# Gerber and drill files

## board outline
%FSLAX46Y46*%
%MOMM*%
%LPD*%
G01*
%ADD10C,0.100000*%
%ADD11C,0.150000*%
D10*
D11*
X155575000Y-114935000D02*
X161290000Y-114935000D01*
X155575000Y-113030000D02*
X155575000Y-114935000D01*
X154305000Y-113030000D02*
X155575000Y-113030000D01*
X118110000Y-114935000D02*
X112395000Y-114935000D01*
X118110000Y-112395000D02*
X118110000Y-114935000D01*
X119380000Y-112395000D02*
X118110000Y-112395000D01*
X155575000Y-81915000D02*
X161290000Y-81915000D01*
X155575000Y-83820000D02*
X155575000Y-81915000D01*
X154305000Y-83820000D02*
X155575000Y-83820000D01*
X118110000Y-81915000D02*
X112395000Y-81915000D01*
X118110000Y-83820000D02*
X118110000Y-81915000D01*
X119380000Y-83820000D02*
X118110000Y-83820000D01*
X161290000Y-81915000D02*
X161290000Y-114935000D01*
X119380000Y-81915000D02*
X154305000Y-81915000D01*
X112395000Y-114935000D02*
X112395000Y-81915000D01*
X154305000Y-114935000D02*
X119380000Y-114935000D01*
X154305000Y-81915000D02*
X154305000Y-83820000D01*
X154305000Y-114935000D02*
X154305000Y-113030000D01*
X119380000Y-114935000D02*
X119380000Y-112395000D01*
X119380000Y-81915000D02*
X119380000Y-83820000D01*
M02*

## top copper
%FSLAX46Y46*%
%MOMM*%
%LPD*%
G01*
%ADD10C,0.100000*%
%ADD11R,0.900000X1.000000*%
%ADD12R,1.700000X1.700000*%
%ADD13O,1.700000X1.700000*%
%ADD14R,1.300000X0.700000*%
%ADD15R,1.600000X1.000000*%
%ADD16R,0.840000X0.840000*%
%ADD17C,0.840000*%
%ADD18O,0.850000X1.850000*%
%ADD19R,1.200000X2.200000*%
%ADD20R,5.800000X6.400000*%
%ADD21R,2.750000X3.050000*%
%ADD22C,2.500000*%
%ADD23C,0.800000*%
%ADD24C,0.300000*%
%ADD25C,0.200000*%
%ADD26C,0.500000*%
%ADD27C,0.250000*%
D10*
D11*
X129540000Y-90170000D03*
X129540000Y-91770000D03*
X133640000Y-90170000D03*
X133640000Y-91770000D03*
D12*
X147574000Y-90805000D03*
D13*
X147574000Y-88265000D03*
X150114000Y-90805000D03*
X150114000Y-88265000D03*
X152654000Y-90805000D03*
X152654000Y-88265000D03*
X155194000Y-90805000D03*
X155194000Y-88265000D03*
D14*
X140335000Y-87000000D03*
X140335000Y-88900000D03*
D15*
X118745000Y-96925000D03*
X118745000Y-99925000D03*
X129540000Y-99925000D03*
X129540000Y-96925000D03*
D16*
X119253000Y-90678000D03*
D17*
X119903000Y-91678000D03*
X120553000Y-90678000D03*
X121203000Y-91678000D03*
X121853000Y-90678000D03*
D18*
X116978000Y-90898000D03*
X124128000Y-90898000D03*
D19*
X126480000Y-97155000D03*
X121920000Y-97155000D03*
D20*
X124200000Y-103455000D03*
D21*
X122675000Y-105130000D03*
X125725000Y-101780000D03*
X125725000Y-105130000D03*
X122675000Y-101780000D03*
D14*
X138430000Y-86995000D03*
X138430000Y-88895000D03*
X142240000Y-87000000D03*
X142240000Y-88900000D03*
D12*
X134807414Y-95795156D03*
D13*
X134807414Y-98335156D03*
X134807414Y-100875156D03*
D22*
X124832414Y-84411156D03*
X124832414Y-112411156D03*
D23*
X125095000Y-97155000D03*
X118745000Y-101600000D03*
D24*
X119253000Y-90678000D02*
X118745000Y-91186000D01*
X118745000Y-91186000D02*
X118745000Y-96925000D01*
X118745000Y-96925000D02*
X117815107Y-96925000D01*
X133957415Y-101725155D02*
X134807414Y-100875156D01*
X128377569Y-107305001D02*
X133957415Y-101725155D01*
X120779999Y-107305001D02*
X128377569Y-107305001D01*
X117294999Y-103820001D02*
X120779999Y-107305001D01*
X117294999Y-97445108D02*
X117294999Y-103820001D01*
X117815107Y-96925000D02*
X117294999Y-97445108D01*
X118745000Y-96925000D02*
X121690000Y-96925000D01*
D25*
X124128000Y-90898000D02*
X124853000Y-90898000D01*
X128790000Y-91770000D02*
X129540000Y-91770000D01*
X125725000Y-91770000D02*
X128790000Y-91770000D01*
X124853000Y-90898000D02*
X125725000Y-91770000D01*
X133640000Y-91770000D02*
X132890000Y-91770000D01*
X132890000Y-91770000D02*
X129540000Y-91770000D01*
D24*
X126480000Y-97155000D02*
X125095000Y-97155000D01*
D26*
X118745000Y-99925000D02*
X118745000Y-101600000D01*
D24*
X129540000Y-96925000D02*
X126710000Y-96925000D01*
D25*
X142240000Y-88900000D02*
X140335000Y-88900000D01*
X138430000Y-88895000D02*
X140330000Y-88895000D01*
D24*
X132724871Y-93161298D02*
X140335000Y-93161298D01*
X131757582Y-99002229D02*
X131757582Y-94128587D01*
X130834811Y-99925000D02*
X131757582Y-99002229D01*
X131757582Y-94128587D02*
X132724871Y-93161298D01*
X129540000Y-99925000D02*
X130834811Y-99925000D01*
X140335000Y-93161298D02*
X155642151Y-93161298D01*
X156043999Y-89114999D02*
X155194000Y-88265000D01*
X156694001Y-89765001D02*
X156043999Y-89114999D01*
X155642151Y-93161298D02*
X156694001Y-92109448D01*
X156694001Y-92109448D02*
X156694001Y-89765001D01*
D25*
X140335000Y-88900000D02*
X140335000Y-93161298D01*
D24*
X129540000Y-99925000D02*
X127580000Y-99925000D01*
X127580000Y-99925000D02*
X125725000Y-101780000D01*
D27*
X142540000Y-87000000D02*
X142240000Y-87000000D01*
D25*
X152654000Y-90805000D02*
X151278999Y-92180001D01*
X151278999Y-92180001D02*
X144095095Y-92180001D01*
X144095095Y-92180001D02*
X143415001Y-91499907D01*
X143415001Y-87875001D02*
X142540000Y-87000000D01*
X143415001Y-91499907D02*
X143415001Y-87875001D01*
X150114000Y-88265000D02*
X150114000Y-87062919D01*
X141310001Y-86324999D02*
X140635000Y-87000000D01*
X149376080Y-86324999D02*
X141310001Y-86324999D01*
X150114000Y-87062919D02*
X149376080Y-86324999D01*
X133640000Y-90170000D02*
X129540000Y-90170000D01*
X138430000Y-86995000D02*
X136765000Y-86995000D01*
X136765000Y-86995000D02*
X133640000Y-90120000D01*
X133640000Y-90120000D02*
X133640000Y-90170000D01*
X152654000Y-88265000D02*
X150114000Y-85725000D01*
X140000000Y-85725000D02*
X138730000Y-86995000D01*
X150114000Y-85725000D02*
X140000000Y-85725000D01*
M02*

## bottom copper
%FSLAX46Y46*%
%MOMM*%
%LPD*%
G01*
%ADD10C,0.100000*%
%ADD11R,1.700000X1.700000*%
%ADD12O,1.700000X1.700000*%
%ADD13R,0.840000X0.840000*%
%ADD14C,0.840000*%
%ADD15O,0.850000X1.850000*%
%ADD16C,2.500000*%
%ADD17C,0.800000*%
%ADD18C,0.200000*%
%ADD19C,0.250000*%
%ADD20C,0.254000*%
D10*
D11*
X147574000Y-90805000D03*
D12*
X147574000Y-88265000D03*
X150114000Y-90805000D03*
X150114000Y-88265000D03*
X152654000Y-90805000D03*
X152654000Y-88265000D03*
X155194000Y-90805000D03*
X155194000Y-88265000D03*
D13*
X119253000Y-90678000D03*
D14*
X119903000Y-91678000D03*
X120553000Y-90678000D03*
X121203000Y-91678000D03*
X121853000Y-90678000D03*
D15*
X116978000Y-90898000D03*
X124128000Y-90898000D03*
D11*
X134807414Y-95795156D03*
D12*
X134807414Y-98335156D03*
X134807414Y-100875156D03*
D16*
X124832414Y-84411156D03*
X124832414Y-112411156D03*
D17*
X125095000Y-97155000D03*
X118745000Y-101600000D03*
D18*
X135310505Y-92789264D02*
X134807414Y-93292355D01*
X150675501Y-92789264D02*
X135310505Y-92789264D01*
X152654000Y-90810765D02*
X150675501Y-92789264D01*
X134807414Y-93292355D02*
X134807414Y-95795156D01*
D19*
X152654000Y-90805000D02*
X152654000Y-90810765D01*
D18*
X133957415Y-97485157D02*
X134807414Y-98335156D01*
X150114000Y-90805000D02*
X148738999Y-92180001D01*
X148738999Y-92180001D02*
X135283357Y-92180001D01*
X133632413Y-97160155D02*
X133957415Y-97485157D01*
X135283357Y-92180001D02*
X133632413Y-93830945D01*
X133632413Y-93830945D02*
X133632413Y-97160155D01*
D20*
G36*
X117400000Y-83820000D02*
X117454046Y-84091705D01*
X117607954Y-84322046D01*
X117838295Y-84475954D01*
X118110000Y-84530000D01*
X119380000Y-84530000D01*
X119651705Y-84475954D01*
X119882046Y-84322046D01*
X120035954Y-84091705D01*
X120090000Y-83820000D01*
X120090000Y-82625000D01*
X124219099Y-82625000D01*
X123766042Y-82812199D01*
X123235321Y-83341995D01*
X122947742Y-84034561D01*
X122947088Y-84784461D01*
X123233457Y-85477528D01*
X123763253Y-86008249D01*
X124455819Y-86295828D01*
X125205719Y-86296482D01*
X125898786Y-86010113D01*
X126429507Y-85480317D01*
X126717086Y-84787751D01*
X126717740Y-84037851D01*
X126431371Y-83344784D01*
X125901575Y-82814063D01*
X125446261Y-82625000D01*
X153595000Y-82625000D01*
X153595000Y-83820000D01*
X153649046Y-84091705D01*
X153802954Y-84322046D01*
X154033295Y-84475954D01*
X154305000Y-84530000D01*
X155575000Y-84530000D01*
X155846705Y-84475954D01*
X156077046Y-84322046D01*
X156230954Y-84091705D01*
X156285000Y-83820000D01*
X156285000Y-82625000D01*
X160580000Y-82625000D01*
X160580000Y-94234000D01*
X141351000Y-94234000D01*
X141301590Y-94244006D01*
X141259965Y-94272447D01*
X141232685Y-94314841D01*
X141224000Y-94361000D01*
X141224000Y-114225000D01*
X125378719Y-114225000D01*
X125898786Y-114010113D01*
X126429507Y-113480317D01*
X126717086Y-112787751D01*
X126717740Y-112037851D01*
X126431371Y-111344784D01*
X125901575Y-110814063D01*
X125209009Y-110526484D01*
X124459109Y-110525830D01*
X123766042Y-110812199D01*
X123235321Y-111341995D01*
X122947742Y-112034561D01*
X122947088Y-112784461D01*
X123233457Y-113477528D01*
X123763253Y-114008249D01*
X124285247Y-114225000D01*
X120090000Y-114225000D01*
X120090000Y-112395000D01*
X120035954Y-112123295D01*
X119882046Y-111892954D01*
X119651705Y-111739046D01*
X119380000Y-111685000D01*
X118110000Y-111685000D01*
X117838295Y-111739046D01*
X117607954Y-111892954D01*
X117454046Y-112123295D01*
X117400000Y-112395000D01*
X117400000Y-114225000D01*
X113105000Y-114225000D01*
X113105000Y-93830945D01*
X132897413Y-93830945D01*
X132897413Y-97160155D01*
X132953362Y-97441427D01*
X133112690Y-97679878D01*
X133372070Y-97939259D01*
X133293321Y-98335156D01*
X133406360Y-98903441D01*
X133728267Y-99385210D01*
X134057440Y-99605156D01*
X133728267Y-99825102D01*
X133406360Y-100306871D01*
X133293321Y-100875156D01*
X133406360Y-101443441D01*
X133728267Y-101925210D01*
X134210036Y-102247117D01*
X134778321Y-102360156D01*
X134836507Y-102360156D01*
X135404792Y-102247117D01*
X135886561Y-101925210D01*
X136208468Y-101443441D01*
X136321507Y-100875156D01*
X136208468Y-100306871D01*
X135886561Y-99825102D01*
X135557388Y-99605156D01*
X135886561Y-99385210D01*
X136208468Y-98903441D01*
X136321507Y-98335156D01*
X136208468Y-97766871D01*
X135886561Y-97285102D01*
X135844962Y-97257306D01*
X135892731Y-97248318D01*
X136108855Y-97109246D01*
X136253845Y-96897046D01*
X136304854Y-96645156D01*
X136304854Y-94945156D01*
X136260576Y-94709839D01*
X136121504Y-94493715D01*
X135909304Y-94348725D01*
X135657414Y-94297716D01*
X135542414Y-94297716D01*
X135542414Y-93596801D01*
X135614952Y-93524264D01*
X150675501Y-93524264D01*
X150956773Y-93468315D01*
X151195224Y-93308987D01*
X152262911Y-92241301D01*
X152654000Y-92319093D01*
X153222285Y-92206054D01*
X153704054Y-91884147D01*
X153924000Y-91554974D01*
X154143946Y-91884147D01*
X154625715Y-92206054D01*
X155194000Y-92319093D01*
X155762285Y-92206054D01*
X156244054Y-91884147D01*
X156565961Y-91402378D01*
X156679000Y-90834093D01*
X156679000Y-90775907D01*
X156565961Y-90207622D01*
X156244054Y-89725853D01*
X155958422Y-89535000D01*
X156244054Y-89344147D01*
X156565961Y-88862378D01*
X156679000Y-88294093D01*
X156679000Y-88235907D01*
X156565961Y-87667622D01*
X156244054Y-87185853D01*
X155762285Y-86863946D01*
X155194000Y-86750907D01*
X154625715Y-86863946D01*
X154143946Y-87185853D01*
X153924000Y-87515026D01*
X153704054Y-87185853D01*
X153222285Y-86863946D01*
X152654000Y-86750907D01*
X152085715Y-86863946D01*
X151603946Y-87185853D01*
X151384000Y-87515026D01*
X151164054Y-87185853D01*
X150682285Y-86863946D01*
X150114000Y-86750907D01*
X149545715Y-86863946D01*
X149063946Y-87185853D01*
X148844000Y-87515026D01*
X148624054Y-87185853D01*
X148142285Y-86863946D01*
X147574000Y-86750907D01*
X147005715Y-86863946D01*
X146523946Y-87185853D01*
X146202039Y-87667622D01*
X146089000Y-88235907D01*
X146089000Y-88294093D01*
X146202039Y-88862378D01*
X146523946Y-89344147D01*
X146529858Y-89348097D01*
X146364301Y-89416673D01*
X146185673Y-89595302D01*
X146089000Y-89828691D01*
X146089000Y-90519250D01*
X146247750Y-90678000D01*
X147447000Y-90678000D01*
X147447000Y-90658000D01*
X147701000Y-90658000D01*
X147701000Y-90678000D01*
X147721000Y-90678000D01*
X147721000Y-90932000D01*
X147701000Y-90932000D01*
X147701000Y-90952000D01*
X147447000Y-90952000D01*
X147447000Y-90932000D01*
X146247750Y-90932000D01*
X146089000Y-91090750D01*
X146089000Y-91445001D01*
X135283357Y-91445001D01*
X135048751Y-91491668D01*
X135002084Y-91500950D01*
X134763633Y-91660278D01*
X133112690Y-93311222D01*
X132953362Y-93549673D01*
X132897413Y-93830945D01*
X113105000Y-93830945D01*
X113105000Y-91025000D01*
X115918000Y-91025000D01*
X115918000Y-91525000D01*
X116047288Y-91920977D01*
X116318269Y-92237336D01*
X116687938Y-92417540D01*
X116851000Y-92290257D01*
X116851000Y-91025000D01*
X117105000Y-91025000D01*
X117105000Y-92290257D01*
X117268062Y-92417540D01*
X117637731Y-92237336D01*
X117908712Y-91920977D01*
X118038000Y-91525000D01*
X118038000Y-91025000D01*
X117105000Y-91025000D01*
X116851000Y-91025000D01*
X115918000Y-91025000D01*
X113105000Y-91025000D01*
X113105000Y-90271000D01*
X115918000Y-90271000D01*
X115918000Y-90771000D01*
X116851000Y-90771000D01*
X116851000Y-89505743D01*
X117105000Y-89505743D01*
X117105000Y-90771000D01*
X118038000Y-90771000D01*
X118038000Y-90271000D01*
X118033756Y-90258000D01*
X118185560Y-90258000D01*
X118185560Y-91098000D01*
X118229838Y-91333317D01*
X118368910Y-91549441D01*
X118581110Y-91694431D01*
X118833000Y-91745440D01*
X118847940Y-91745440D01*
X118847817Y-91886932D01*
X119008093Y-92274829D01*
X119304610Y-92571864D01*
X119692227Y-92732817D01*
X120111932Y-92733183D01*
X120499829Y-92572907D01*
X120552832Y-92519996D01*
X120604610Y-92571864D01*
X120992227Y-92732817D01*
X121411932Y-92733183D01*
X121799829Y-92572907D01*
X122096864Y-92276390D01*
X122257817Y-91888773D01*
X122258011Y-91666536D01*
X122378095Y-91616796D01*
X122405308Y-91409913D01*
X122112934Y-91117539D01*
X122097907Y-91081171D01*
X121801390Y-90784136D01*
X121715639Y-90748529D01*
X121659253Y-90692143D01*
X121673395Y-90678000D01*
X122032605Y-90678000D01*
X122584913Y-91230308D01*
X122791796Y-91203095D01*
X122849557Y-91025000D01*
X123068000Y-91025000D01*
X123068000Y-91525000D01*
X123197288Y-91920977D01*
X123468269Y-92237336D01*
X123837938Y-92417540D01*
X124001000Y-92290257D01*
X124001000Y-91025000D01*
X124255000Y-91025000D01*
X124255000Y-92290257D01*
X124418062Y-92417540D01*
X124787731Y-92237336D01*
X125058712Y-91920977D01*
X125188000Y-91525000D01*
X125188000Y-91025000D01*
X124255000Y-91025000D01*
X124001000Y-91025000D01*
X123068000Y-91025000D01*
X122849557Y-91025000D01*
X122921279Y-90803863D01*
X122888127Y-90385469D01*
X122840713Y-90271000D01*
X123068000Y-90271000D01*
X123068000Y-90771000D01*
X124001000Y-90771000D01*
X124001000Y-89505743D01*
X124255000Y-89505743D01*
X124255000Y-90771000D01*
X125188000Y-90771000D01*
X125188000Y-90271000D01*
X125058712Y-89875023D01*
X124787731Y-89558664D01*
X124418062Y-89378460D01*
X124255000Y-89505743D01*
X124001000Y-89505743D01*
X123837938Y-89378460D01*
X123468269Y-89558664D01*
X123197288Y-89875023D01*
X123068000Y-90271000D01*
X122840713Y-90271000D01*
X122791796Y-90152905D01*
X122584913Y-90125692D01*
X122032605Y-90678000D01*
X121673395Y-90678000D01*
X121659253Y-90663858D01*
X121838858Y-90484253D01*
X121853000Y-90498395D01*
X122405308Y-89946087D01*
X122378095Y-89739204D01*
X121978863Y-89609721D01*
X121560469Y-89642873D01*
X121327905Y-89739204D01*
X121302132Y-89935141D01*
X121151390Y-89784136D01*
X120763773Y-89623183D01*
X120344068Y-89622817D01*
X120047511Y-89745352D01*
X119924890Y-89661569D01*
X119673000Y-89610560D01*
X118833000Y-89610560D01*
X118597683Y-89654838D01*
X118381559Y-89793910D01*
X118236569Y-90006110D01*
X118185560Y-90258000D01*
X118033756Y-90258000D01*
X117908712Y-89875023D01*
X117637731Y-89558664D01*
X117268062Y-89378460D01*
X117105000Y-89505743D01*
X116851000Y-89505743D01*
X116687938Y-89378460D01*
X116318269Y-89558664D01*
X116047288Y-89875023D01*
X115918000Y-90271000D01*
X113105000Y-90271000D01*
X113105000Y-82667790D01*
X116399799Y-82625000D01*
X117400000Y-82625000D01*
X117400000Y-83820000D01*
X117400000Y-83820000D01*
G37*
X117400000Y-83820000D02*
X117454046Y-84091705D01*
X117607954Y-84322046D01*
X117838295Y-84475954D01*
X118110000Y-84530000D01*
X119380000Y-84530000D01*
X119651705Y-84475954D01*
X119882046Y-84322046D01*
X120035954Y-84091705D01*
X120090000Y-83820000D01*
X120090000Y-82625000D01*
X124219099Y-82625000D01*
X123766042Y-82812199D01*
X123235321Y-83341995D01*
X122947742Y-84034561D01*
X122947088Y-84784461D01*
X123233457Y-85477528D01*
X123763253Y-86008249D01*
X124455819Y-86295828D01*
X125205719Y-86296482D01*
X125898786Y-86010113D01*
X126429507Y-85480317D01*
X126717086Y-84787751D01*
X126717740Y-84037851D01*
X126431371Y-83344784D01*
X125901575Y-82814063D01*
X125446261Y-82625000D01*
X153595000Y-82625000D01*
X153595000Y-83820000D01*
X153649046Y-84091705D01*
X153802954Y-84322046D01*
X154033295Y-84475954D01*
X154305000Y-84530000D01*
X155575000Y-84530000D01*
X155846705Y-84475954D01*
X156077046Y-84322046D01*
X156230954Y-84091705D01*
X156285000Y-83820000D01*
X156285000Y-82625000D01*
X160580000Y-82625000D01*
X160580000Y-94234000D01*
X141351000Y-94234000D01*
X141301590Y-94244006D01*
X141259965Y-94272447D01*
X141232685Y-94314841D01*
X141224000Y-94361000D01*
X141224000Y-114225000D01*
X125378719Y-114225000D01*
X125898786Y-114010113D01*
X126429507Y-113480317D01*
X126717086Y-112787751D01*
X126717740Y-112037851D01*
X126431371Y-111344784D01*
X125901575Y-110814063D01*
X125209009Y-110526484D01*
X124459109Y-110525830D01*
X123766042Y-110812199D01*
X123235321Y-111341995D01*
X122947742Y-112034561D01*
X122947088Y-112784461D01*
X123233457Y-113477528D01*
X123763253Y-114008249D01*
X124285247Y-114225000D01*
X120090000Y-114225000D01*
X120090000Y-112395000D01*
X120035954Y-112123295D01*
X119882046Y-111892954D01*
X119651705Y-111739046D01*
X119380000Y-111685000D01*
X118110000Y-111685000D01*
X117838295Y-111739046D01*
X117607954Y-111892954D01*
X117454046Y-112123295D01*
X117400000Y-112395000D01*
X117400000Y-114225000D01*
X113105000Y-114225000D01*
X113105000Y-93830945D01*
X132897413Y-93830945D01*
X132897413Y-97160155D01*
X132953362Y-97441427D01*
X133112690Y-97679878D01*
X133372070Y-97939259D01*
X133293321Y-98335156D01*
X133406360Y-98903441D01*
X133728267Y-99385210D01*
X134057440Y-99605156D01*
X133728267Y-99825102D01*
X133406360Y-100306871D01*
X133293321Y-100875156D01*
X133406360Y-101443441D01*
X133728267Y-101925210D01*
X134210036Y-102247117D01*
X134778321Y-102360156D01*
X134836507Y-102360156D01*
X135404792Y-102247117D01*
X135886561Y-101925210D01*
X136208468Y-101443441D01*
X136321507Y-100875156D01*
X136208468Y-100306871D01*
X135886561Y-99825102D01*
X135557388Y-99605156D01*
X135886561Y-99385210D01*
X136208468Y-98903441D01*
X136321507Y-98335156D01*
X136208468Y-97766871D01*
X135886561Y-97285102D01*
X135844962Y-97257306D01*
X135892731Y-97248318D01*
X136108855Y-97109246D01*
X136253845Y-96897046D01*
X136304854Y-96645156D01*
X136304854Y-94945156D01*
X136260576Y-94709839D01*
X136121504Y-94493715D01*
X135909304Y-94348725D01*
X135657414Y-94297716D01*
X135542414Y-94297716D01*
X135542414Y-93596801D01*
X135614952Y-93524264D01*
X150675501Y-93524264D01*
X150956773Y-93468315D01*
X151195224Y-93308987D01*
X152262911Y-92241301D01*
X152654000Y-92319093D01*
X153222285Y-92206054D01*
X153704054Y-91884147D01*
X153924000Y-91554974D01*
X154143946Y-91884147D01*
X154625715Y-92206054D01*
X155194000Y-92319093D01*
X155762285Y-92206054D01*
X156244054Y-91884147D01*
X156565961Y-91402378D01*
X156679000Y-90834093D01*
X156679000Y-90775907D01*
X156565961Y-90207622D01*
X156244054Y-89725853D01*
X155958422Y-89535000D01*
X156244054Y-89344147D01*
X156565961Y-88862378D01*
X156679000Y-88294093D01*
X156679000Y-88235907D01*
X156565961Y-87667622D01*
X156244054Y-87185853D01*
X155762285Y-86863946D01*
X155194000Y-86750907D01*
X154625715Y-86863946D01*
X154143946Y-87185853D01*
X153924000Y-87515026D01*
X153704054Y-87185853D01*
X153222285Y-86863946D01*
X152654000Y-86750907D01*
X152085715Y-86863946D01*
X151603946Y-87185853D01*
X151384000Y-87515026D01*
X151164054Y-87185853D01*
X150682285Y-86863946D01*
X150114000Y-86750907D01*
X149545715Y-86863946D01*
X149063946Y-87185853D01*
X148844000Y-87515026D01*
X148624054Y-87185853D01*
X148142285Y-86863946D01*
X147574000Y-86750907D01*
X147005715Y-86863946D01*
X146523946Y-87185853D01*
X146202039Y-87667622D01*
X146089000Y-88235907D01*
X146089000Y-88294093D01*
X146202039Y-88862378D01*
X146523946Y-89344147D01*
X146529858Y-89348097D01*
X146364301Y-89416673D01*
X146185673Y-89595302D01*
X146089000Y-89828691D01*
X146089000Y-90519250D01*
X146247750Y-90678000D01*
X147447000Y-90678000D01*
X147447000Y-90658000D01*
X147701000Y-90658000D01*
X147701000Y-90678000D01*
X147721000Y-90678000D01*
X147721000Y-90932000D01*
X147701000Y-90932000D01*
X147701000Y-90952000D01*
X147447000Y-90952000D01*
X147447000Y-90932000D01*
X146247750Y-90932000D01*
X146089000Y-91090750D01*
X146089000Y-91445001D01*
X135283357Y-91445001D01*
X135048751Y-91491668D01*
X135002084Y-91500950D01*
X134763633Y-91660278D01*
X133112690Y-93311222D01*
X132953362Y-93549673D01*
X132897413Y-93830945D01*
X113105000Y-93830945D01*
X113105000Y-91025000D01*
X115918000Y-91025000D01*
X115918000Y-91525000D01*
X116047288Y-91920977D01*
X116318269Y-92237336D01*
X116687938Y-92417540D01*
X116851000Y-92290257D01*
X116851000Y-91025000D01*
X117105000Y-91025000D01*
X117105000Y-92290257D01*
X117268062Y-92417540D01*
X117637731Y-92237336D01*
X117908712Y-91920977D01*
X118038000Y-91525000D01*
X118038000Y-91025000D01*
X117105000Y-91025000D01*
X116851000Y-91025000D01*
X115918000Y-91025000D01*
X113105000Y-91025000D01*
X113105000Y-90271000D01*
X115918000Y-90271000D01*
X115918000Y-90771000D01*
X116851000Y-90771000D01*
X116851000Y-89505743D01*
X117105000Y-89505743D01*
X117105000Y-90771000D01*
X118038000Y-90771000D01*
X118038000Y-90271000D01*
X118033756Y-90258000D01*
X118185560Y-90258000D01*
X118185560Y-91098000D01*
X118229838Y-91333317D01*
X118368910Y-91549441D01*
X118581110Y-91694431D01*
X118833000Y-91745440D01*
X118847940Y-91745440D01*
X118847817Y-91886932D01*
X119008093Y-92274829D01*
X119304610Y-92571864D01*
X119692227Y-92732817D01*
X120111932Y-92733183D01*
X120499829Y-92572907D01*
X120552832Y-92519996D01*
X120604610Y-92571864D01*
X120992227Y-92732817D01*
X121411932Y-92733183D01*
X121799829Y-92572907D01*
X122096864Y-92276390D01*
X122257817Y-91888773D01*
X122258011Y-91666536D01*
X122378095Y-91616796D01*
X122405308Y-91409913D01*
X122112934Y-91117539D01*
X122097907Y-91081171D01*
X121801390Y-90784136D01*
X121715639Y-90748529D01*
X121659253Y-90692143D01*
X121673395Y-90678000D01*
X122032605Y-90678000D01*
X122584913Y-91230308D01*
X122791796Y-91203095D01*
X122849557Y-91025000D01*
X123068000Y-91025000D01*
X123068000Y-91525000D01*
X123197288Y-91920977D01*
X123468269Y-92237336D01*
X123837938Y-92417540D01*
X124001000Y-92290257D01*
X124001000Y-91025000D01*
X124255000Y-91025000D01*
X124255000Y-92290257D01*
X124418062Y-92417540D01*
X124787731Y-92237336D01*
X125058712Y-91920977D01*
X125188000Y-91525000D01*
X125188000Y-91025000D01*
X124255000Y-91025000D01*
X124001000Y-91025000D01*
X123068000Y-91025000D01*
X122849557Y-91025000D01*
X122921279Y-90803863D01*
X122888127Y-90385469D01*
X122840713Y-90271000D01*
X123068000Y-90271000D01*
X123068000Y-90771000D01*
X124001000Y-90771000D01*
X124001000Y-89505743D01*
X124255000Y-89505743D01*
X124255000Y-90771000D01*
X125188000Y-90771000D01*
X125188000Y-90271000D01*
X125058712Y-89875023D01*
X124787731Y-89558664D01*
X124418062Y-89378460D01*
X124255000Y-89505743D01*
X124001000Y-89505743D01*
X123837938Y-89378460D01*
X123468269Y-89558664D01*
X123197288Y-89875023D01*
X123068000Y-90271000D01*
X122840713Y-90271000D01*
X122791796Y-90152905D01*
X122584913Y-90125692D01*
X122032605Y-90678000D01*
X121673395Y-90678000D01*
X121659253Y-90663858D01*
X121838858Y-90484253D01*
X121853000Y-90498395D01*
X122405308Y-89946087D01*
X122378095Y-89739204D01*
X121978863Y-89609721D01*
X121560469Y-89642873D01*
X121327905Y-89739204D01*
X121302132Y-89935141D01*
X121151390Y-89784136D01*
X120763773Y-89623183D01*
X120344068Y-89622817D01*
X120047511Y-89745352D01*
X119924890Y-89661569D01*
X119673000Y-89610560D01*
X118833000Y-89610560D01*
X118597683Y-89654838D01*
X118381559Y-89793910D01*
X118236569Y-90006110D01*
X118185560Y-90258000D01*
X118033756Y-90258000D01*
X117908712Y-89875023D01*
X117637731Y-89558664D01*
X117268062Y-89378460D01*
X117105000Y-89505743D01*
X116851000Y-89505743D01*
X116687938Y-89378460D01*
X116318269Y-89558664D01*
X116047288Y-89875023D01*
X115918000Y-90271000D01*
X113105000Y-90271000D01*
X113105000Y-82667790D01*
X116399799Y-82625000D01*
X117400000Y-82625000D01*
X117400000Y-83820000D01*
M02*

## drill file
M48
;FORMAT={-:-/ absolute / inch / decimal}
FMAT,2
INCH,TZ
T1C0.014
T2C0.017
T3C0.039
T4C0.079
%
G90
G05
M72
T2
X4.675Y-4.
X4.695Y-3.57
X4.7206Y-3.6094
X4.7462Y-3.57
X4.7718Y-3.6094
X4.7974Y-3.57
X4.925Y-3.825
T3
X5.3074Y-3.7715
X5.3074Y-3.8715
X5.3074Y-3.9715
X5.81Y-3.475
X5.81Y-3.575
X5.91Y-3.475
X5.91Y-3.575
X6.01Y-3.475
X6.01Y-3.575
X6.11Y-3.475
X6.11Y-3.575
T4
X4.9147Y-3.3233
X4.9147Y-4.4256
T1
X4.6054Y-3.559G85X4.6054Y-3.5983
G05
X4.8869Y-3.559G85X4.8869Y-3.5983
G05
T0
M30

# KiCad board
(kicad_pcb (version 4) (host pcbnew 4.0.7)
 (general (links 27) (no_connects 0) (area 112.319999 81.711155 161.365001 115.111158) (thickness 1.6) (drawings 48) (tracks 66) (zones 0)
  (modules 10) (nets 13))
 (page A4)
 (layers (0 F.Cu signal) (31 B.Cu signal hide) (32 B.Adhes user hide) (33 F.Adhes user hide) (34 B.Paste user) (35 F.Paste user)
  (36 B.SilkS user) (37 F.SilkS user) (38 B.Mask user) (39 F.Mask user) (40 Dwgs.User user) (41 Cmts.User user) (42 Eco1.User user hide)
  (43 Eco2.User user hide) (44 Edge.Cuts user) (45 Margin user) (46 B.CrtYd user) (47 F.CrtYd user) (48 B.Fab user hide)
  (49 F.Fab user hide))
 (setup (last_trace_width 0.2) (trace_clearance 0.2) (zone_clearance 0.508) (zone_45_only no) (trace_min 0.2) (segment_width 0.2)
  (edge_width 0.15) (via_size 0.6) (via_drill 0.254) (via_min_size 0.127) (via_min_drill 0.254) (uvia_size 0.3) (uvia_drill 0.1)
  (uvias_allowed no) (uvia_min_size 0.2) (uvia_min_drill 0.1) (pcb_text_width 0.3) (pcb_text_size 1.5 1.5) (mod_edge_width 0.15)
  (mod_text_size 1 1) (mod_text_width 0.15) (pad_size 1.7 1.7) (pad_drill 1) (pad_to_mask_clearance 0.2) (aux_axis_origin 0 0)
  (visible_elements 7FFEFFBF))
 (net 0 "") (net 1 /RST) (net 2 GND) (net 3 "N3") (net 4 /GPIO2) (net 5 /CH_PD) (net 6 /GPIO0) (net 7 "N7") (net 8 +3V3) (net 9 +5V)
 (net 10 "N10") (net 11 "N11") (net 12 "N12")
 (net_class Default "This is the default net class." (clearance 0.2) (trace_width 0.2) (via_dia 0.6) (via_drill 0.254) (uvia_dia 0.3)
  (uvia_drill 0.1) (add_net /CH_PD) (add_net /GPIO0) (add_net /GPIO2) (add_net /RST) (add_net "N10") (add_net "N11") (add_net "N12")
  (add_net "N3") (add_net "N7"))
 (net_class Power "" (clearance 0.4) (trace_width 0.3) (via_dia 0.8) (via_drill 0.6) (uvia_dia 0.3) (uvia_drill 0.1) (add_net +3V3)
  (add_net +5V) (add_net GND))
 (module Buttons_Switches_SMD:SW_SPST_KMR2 (layer F.Cu) (at 131.59 90.97)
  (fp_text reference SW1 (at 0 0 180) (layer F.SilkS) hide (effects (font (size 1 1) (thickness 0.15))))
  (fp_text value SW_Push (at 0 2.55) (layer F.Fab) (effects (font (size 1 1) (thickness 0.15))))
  (pad 1 smd rect (at -2.05 -0.8) (size 0.9 1) (layers F.Cu F.Paste F.Mask) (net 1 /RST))
  (pad 2 smd rect (at -2.05 0.8) (size 0.9 1) (layers F.Cu F.Paste F.Mask) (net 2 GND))
  (pad 1 smd rect (at 2.05 -0.8) (size 0.9 1) (layers F.Cu F.Paste F.Mask) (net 1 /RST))
  (pad 2 smd rect (at 2.05 0.8) (size 0.9 1) (layers F.Cu F.Paste F.Mask) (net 2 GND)))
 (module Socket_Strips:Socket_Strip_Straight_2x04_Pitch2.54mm (layer B.Cu) (at 147.574 90.805 270)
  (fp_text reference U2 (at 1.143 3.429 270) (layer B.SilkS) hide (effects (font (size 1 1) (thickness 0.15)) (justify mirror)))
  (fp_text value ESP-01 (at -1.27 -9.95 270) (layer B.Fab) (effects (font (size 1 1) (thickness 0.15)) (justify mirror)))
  (pad 1 thru_hole rect (at 0 0 270) (size 1.7 1.7) (drill 1) (layers *.Cu *.Mask) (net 2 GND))
  (pad 2 thru_hole oval (at -2.54 0 270) (size 1.7 1.7) (drill 1) (layers *.Cu *.Mask) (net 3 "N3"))
  (pad 3 thru_hole oval (at 0 -2.54 270) (size 1.7 1.7) (drill 1) (layers *.Cu *.Mask) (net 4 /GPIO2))
  (pad 4 thru_hole oval (at -2.54 -2.54 270) (size 1.7 1.7) (drill 1) (layers *.Cu *.Mask) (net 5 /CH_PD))
  (pad 5 thru_hole oval (at 0 -5.08 270) (size 1.7 1.7) (drill 1) (layers *.Cu *.Mask) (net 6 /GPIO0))
  (pad 6 thru_hole oval (at -2.54 -5.08 270) (size 1.7 1.7) (drill 1) (layers *.Cu *.Mask) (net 1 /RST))
  (pad 7 thru_hole oval (at 0 -7.62 270) (size 1.7 1.7) (drill 1) (layers *.Cu *.Mask) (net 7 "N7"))
  (pad 8 thru_hole oval (at -2.54 -7.62 270) (size 1.7 1.7) (drill 1) (layers *.Cu *.Mask) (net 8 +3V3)))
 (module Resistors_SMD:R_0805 (layer F.Cu) (at 140.335 87.95 270)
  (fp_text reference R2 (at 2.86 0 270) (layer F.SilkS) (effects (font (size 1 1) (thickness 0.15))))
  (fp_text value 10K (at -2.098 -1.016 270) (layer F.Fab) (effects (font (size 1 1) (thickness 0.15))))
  (pad 1 smd rect (at -0.95 0 270) (size 0.7 1.3) (layers F.Cu F.Paste F.Mask) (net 5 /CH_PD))
  (pad 2 smd rect (at 0.95 0 270) (size 0.7 1.3) (layers F.Cu F.Paste F.Mask) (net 8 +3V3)))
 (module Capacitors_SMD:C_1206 (layer F.Cu) (at 118.745 98.425 270)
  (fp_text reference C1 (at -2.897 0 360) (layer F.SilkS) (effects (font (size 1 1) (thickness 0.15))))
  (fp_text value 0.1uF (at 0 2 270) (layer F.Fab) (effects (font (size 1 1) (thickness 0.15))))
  (pad 1 smd rect (at -1.5 0 270) (size 1 1.6) (layers F.Cu F.Paste F.Mask) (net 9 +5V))
  (pad 2 smd rect (at 1.5 0 270) (size 1 1.6) (layers F.Cu F.Paste F.Mask) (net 2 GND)))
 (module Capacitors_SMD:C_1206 (layer F.Cu) (at 129.54 98.425 90)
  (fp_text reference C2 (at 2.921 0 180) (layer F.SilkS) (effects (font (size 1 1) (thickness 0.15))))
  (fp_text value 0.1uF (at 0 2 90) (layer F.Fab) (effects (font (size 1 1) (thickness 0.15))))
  (pad 1 smd rect (at -1.5 0 90) (size 1 1.6) (layers F.Cu F.Paste F.Mask) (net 8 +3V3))
  (pad 2 smd rect (at 1.5 0 90) (size 1 1.6) (layers F.Cu F.Paste F.Mask) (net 2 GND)))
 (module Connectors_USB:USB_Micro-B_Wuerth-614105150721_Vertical (layer F.Cu) (at 119.253 90.678)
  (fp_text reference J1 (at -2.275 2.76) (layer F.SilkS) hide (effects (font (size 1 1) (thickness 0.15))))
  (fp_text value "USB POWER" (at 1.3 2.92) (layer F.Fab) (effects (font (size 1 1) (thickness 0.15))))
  (pad 1 thru_hole rect (at 0 0) (size 0.84 0.84) (drill 0.44) (layers *.Cu *.Mask) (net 9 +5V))
  (pad 2 thru_hole circle (at 0.65 1) (size 0.84 0.84) (drill 0.44) (layers *.Cu *.Mask) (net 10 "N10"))
  (pad 3 thru_hole circle (at 1.3 0) (size 0.84 0.84) (drill 0.44) (layers *.Cu *.Mask) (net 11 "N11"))
  (pad 4 thru_hole circle (at 1.95 1) (size 0.84 0.84) (drill 0.44) (layers *.Cu *.Mask) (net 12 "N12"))
  (pad 5 thru_hole circle (at 2.6 0) (size 0.84 0.84) (drill 0.44) (layers *.Cu *.Mask) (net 2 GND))
  (pad 6 thru_hole oval (at -2.275 0.22) (size 0.85 1.85) (drill oval 0.35 1.35) (layers *.Cu *.Mask) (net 2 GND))
  (pad 6 thru_hole oval (at 4.875 0.22) (size 0.85 1.85) (drill oval 0.35 1.35) (layers *.Cu *.Mask) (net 2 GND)))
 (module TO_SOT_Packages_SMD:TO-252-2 (layer F.Cu) (at 124.2 101.355 270)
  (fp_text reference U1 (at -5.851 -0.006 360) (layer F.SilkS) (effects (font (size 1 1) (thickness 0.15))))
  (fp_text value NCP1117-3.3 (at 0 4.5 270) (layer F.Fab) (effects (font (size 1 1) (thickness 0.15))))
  (pad 1 smd rect (at -4.2 -2.28 270) (size 2.2 1.2) (layers F.Cu F.Paste F.Mask) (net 2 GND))
  (pad 3 smd rect (at -4.2 2.28 270) (size 2.2 1.2) (layers F.Cu F.Paste F.Mask) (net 9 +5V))
  (pad 2 smd rect (at 2.1 0 270) (size 6.4 5.8) (layers F.Cu F.Mask) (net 8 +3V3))
  (pad 2 smd rect (at 3.775 1.525 270) (size 3.05 2.75) (layers F.Cu F.Paste) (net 8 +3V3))
  (pad 2 smd rect (at 0.425 -1.525 270) (size 3.05 2.75) (layers F.Cu F.Paste) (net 8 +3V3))
  (pad 2 smd rect (at 3.775 -1.525 270) (size 3.05 2.75) (layers F.Cu F.Paste) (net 8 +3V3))
  (pad 2 smd rect (at 0.425 1.525 270) (size 3.05 2.75) (layers F.Cu F.Paste) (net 8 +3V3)))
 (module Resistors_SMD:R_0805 (layer F.Cu) (at 138.43 87.945 270)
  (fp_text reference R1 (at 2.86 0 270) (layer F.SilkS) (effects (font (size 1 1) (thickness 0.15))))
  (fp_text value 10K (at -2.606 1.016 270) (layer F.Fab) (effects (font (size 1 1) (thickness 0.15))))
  (pad 1 smd rect (at -0.95 0 270) (size 0.7 1.3) (layers F.Cu F.Paste F.Mask) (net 1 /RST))
  (pad 2 smd rect (at 0.95 0 270) (size 0.7 1.3) (layers F.Cu F.Paste F.Mask) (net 8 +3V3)))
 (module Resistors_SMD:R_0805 (layer F.Cu) (at 142.24 87.95 270)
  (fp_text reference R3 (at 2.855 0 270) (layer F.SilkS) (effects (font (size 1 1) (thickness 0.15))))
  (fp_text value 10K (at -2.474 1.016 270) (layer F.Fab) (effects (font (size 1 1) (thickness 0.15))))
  (pad 1 smd rect (at -0.95 0 270) (size 0.7 1.3) (layers F.Cu F.Paste F.Mask) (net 6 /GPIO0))
  (pad 2 smd rect (at 0.95 0 270) (size 0.7 1.3) (layers F.Cu F.Paste F.Mask) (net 8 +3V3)))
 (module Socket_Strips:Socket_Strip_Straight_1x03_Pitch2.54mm (layer B.Cu) (at 134.807414 95.795156 180)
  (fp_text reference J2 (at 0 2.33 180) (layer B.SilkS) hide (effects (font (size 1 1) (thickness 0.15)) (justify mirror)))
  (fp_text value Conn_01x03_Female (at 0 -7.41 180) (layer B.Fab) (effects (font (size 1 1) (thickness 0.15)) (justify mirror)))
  (pad 1 thru_hole rect (at 0 0 180) (size 1.7 1.7) (drill 1) (layers *.Cu *.Mask) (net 6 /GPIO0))
  (pad 2 thru_hole oval (at 0 -2.54 180) (size 1.7 1.7) (drill 1) (layers *.Cu *.Mask) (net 4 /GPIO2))
  (pad 3 thru_hole oval (at 0 -5.08 180) (size 1.7 1.7) (drill 1) (layers *.Cu *.Mask) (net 9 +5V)))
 (gr_line (start 155.575 114.935) (end 161.29 114.935) (layer Edge.Cuts) (width 0.15))
 (gr_line (start 155.575 113.03) (end 155.575 114.935) (layer Edge.Cuts) (width 0.15))
 (gr_line (start 154.305 113.03) (end 155.575 113.03) (layer Edge.Cuts) (width 0.15))
 (gr_line (start 118.11 114.935) (end 112.395 114.935) (layer Edge.Cuts) (width 0.15))
 (gr_line (start 118.11 112.395) (end 118.11 114.935) (layer Edge.Cuts) (width 0.15))
 (gr_line (start 119.38 112.395) (end 118.11 112.395) (layer Edge.Cuts) (width 0.15))
 (gr_line (start 155.575 81.915) (end 161.29 81.915) (layer Edge.Cuts) (width 0.15))
 (gr_line (start 155.575 83.82) (end 155.575 81.915) (layer Edge.Cuts) (width 0.15))
 (gr_line (start 154.305 83.82) (end 155.575 83.82) (layer Edge.Cuts) (width 0.15))
 (gr_line (start 118.11 81.915) (end 112.395 81.915) (layer Edge.Cuts) (width 0.15))
 (gr_line (start 118.11 83.82) (end 118.11 81.915) (layer Edge.Cuts) (width 0.15))
 (gr_line (start 119.38 83.82) (end 118.11 83.82) (layer Edge.Cuts) (width 0.15))
 (gr_line (start 161.29 81.915) (end 161.29 114.935) (layer Edge.Cuts) (width 0.15))
 (gr_line (start 119.38 81.915) (end 154.305 81.915) (layer Edge.Cuts) (width 0.15))
 (gr_line (start 112.395 114.935) (end 112.395 81.915) (layer Edge.Cuts) (width 0.15))
 (gr_line (start 154.305 114.935) (end 119.38 114.935) (layer Edge.Cuts) (width 0.15))
 (gr_line (start 154.305 81.915) (end 154.305 83.82) (layer Edge.Cuts) (width 0.15))
 (gr_line (start 154.305 114.935) (end 154.305 113.03) (layer Edge.Cuts) (width 0.15))
 (gr_line (start 119.38 114.935) (end 119.38 112.395) (layer Edge.Cuts) (width 0.15))
 (gr_line (start 119.38 81.915) (end 119.38 83.82) (layer Edge.Cuts) (width 0.15))
 (via (at 124.832414 84.411156) (size 2.5) (drill 2) (layers F.Cu B.Cu) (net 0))
 (via (at 124.832414 112.411156) (size 2.5) (drill 2) (layers F.Cu B.Cu) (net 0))
 (segment (start 119.253 90.678) (end 118.745 91.186) (width 0.3) (layer F.Cu) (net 9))
 (segment (start 118.745 91.186) (end 118.745 96.925) (width 0.3) (layer F.Cu) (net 9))
 (segment (start 118.745 96.925) (end 117.815107 96.925) (width 0.3) (layer F.Cu) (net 9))
 (segment (start 133.957415 101.725155) (end 134.807414 100.875156) (width 0.3) (layer F.Cu) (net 9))
 (segment (start 128.377569 107.305001) (end 133.957415 101.725155) (width 0.3) (layer F.Cu) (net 9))
 (segment (start 120.779999 107.305001) (end 128.377569 107.305001) (width 0.3) (layer F.Cu) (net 9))
 (segment (start 117.294999 103.820001) (end 120.779999 107.305001) (width 0.3) (layer F.Cu) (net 9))
 (segment (start 117.294999 97.445108) (end 117.294999 103.820001) (width 0.3) (layer F.Cu) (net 9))
 (segment (start 117.815107 96.925) (end 117.294999 97.445108) (width 0.3) (layer F.Cu) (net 9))
 (segment (start 118.745 96.925) (end 121.69 96.925) (width 0.3) (layer F.Cu) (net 9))
 (segment (start 124.128 90.898) (end 124.853 90.898) (width 0.2) (layer F.Cu) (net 2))
 (segment (start 128.79 91.77) (end 129.54 91.77) (width 0.2) (layer F.Cu) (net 2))
 (segment (start 125.725 91.77) (end 128.79 91.77) (width 0.2) (layer F.Cu) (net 2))
 (segment (start 124.853 90.898) (end 125.725 91.77) (width 0.2) (layer F.Cu) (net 2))
 (segment (start 133.64 91.77) (end 132.89 91.77) (width 0.2) (layer F.Cu) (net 2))
 (segment (start 132.89 91.77) (end 129.54 91.77) (width 0.2) (layer F.Cu) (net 2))
 (segment (start 126.48 97.155) (end 125.095 97.155) (width 0.3) (layer F.Cu) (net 2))
 (via (at 125.095 97.155) (size 0.8) (drill 0.44) (layers F.Cu B.Cu) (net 2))
 (segment (start 118.745 99.925) (end 118.745 101.6) (width 0.5) (layer F.Cu) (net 2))
 (via (at 118.745 101.6) (size 0.8) (drill 0.44) (layers F.Cu B.Cu) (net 2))
 (segment (start 129.54 96.925) (end 126.71 96.925) (width 0.3) (layer F.Cu) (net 2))
 (segment (start 142.24 88.9) (end 140.335 88.9) (width 0.2) (layer F.Cu) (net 8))
 (segment (start 138.43 88.895) (end 140.33 88.895) (width 0.2) (layer F.Cu) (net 8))
 (segment (start 132.724871 93.161298) (end 140.335 93.161298) (width 0.3) (layer F.Cu) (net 8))
 (segment (start 131.757582 99.002229) (end 131.757582 94.128587) (width 0.3) (layer F.Cu) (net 8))
 (segment (start 130.834811 99.925) (end 131.757582 99.002229) (width 0.3) (layer F.Cu) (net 8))
 (segment (start 131.757582 94.128587) (end 132.724871 93.161298) (width 0.3) (layer F.Cu) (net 8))
 (segment (start 129.54 99.925) (end 130.834811 99.925) (width 0.3) (layer F.Cu) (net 8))
 (segment (start 140.335 93.161298) (end 155.642151 93.161298) (width 0.3) (layer F.Cu) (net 8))
 (segment (start 156.043999 89.114999) (end 155.194 88.265) (width 0.3) (layer F.Cu) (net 8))
 (segment (start 156.694001 89.765001) (end 156.043999 89.114999) (width 0.3) (layer F.Cu) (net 8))
 (segment (start 155.642151 93.161298) (end 156.694001 92.109448) (width 0.3) (layer F.Cu) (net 8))
 (segment (start 156.694001 92.109448) (end 156.694001 89.765001) (width 0.3) (layer F.Cu) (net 8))
 (segment (start 140.335 88.9) (end 140.335 93.161298) (width 0.2) (layer F.Cu) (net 8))
 (segment (start 129.54 99.925) (end 127.58 99.925) (width 0.3) (layer F.Cu) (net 8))
 (segment (start 127.58 99.925) (end 125.725 101.78) (width 0.3) (layer F.Cu) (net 8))
 (segment (start 142.54 87) (end 142.24 87) (width 0.25) (layer F.Cu) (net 6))
 (segment (start 152.654 90.805) (end 151.278999 92.180001) (width 0.2) (layer F.Cu) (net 6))
 (segment (start 151.278999 92.180001) (end 144.095095 92.180001) (width 0.2) (layer F.Cu) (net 6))
 (segment (start 144.095095 92.180001) (end 143.415001 91.499907) (width 0.2) (layer F.Cu) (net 6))
 (segment (start 143.415001 87.875001) (end 142.54 87) (width 0.2) (layer F.Cu) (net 6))
 (segment (start 143.415001 91.499907) (end 143.415001 87.875001) (width 0.2) (layer F.Cu) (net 6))
 (segment (start 135.310505 92.789264) (end 134.807414 93.292355) (width 0.2) (layer B.Cu) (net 6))
 (segment (start 150.675501 92.789264) (end 135.310505 92.789264) (width 0.2) (layer B.Cu) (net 6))
 (segment (start 152.654 90.810765) (end 150.675501 92.789264) (width 0.2) (layer B.Cu) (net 6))
 (segment (start 134.807414 93.292355) (end 134.807414 95.795156) (width 0.2) (layer B.Cu) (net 6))
 (segment (start 152.654 90.805) (end 152.654 90.810765) (width 0.25) (layer B.Cu) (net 6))
 (segment (start 150.114 88.265) (end 150.114 87.062919) (width 0.2) (layer F.Cu) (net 5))
 (segment (start 141.310001 86.324999) (end 140.635 87) (width 0.2) (layer F.Cu) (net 5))
 (segment (start 149.37608 86.324999) (end 141.310001 86.324999) (width 0.2) (layer F.Cu) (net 5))
 (segment (start 150.114 87.062919) (end 149.37608 86.324999) (width 0.2) (layer F.Cu) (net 5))
 (segment (start 133.957415 97.485157) (end 134.807414 98.335156) (width 0.2) (layer B.Cu) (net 4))
 (segment (start 150.114 90.805) (end 148.738999 92.180001) (width 0.2) (layer B.Cu) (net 4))
 (segment (start 148.738999 92.180001) (end 135.283357 92.180001) (width 0.2) (layer B.Cu) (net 4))
 (segment (start 133.632413 97.160155) (end 133.957415 97.485157) (width 0.2) (layer B.Cu) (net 4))
 (segment (start 135.283357 92.180001) (end 133.632413 93.830945) (width 0.2) (layer B.Cu) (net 4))
 (segment (start 133.632413 93.830945) (end 133.632413 97.160155) (width 0.2) (layer B.Cu) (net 4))
 (segment (start 133.64 90.17) (end 129.54 90.17) (width 0.2) (layer F.Cu) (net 1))
 (segment (start 138.43 86.995) (end 136.765 86.995) (width 0.2) (layer F.Cu) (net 1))
 (segment (start 136.765 86.995) (end 133.64 90.12) (width 0.2) (layer F.Cu) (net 1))
 (segment (start 133.64 90.12) (end 133.64 90.17) (width 0.2) (layer F.Cu) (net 1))
 (segment (start 152.654 88.265) (end 150.114 85.725) (width 0.2) (layer F.Cu) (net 1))
 (segment (start 140 85.725) (end 138.73 86.995) (width 0.2) (layer F.Cu) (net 1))
 (segment (start 150.114 85.725) (end 140 85.725) (width 0.2) (layer F.Cu) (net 1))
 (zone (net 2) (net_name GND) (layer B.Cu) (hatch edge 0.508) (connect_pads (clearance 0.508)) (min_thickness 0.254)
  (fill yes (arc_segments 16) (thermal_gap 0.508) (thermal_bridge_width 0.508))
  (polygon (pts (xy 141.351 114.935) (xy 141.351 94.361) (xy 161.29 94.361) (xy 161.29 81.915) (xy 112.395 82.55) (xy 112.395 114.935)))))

